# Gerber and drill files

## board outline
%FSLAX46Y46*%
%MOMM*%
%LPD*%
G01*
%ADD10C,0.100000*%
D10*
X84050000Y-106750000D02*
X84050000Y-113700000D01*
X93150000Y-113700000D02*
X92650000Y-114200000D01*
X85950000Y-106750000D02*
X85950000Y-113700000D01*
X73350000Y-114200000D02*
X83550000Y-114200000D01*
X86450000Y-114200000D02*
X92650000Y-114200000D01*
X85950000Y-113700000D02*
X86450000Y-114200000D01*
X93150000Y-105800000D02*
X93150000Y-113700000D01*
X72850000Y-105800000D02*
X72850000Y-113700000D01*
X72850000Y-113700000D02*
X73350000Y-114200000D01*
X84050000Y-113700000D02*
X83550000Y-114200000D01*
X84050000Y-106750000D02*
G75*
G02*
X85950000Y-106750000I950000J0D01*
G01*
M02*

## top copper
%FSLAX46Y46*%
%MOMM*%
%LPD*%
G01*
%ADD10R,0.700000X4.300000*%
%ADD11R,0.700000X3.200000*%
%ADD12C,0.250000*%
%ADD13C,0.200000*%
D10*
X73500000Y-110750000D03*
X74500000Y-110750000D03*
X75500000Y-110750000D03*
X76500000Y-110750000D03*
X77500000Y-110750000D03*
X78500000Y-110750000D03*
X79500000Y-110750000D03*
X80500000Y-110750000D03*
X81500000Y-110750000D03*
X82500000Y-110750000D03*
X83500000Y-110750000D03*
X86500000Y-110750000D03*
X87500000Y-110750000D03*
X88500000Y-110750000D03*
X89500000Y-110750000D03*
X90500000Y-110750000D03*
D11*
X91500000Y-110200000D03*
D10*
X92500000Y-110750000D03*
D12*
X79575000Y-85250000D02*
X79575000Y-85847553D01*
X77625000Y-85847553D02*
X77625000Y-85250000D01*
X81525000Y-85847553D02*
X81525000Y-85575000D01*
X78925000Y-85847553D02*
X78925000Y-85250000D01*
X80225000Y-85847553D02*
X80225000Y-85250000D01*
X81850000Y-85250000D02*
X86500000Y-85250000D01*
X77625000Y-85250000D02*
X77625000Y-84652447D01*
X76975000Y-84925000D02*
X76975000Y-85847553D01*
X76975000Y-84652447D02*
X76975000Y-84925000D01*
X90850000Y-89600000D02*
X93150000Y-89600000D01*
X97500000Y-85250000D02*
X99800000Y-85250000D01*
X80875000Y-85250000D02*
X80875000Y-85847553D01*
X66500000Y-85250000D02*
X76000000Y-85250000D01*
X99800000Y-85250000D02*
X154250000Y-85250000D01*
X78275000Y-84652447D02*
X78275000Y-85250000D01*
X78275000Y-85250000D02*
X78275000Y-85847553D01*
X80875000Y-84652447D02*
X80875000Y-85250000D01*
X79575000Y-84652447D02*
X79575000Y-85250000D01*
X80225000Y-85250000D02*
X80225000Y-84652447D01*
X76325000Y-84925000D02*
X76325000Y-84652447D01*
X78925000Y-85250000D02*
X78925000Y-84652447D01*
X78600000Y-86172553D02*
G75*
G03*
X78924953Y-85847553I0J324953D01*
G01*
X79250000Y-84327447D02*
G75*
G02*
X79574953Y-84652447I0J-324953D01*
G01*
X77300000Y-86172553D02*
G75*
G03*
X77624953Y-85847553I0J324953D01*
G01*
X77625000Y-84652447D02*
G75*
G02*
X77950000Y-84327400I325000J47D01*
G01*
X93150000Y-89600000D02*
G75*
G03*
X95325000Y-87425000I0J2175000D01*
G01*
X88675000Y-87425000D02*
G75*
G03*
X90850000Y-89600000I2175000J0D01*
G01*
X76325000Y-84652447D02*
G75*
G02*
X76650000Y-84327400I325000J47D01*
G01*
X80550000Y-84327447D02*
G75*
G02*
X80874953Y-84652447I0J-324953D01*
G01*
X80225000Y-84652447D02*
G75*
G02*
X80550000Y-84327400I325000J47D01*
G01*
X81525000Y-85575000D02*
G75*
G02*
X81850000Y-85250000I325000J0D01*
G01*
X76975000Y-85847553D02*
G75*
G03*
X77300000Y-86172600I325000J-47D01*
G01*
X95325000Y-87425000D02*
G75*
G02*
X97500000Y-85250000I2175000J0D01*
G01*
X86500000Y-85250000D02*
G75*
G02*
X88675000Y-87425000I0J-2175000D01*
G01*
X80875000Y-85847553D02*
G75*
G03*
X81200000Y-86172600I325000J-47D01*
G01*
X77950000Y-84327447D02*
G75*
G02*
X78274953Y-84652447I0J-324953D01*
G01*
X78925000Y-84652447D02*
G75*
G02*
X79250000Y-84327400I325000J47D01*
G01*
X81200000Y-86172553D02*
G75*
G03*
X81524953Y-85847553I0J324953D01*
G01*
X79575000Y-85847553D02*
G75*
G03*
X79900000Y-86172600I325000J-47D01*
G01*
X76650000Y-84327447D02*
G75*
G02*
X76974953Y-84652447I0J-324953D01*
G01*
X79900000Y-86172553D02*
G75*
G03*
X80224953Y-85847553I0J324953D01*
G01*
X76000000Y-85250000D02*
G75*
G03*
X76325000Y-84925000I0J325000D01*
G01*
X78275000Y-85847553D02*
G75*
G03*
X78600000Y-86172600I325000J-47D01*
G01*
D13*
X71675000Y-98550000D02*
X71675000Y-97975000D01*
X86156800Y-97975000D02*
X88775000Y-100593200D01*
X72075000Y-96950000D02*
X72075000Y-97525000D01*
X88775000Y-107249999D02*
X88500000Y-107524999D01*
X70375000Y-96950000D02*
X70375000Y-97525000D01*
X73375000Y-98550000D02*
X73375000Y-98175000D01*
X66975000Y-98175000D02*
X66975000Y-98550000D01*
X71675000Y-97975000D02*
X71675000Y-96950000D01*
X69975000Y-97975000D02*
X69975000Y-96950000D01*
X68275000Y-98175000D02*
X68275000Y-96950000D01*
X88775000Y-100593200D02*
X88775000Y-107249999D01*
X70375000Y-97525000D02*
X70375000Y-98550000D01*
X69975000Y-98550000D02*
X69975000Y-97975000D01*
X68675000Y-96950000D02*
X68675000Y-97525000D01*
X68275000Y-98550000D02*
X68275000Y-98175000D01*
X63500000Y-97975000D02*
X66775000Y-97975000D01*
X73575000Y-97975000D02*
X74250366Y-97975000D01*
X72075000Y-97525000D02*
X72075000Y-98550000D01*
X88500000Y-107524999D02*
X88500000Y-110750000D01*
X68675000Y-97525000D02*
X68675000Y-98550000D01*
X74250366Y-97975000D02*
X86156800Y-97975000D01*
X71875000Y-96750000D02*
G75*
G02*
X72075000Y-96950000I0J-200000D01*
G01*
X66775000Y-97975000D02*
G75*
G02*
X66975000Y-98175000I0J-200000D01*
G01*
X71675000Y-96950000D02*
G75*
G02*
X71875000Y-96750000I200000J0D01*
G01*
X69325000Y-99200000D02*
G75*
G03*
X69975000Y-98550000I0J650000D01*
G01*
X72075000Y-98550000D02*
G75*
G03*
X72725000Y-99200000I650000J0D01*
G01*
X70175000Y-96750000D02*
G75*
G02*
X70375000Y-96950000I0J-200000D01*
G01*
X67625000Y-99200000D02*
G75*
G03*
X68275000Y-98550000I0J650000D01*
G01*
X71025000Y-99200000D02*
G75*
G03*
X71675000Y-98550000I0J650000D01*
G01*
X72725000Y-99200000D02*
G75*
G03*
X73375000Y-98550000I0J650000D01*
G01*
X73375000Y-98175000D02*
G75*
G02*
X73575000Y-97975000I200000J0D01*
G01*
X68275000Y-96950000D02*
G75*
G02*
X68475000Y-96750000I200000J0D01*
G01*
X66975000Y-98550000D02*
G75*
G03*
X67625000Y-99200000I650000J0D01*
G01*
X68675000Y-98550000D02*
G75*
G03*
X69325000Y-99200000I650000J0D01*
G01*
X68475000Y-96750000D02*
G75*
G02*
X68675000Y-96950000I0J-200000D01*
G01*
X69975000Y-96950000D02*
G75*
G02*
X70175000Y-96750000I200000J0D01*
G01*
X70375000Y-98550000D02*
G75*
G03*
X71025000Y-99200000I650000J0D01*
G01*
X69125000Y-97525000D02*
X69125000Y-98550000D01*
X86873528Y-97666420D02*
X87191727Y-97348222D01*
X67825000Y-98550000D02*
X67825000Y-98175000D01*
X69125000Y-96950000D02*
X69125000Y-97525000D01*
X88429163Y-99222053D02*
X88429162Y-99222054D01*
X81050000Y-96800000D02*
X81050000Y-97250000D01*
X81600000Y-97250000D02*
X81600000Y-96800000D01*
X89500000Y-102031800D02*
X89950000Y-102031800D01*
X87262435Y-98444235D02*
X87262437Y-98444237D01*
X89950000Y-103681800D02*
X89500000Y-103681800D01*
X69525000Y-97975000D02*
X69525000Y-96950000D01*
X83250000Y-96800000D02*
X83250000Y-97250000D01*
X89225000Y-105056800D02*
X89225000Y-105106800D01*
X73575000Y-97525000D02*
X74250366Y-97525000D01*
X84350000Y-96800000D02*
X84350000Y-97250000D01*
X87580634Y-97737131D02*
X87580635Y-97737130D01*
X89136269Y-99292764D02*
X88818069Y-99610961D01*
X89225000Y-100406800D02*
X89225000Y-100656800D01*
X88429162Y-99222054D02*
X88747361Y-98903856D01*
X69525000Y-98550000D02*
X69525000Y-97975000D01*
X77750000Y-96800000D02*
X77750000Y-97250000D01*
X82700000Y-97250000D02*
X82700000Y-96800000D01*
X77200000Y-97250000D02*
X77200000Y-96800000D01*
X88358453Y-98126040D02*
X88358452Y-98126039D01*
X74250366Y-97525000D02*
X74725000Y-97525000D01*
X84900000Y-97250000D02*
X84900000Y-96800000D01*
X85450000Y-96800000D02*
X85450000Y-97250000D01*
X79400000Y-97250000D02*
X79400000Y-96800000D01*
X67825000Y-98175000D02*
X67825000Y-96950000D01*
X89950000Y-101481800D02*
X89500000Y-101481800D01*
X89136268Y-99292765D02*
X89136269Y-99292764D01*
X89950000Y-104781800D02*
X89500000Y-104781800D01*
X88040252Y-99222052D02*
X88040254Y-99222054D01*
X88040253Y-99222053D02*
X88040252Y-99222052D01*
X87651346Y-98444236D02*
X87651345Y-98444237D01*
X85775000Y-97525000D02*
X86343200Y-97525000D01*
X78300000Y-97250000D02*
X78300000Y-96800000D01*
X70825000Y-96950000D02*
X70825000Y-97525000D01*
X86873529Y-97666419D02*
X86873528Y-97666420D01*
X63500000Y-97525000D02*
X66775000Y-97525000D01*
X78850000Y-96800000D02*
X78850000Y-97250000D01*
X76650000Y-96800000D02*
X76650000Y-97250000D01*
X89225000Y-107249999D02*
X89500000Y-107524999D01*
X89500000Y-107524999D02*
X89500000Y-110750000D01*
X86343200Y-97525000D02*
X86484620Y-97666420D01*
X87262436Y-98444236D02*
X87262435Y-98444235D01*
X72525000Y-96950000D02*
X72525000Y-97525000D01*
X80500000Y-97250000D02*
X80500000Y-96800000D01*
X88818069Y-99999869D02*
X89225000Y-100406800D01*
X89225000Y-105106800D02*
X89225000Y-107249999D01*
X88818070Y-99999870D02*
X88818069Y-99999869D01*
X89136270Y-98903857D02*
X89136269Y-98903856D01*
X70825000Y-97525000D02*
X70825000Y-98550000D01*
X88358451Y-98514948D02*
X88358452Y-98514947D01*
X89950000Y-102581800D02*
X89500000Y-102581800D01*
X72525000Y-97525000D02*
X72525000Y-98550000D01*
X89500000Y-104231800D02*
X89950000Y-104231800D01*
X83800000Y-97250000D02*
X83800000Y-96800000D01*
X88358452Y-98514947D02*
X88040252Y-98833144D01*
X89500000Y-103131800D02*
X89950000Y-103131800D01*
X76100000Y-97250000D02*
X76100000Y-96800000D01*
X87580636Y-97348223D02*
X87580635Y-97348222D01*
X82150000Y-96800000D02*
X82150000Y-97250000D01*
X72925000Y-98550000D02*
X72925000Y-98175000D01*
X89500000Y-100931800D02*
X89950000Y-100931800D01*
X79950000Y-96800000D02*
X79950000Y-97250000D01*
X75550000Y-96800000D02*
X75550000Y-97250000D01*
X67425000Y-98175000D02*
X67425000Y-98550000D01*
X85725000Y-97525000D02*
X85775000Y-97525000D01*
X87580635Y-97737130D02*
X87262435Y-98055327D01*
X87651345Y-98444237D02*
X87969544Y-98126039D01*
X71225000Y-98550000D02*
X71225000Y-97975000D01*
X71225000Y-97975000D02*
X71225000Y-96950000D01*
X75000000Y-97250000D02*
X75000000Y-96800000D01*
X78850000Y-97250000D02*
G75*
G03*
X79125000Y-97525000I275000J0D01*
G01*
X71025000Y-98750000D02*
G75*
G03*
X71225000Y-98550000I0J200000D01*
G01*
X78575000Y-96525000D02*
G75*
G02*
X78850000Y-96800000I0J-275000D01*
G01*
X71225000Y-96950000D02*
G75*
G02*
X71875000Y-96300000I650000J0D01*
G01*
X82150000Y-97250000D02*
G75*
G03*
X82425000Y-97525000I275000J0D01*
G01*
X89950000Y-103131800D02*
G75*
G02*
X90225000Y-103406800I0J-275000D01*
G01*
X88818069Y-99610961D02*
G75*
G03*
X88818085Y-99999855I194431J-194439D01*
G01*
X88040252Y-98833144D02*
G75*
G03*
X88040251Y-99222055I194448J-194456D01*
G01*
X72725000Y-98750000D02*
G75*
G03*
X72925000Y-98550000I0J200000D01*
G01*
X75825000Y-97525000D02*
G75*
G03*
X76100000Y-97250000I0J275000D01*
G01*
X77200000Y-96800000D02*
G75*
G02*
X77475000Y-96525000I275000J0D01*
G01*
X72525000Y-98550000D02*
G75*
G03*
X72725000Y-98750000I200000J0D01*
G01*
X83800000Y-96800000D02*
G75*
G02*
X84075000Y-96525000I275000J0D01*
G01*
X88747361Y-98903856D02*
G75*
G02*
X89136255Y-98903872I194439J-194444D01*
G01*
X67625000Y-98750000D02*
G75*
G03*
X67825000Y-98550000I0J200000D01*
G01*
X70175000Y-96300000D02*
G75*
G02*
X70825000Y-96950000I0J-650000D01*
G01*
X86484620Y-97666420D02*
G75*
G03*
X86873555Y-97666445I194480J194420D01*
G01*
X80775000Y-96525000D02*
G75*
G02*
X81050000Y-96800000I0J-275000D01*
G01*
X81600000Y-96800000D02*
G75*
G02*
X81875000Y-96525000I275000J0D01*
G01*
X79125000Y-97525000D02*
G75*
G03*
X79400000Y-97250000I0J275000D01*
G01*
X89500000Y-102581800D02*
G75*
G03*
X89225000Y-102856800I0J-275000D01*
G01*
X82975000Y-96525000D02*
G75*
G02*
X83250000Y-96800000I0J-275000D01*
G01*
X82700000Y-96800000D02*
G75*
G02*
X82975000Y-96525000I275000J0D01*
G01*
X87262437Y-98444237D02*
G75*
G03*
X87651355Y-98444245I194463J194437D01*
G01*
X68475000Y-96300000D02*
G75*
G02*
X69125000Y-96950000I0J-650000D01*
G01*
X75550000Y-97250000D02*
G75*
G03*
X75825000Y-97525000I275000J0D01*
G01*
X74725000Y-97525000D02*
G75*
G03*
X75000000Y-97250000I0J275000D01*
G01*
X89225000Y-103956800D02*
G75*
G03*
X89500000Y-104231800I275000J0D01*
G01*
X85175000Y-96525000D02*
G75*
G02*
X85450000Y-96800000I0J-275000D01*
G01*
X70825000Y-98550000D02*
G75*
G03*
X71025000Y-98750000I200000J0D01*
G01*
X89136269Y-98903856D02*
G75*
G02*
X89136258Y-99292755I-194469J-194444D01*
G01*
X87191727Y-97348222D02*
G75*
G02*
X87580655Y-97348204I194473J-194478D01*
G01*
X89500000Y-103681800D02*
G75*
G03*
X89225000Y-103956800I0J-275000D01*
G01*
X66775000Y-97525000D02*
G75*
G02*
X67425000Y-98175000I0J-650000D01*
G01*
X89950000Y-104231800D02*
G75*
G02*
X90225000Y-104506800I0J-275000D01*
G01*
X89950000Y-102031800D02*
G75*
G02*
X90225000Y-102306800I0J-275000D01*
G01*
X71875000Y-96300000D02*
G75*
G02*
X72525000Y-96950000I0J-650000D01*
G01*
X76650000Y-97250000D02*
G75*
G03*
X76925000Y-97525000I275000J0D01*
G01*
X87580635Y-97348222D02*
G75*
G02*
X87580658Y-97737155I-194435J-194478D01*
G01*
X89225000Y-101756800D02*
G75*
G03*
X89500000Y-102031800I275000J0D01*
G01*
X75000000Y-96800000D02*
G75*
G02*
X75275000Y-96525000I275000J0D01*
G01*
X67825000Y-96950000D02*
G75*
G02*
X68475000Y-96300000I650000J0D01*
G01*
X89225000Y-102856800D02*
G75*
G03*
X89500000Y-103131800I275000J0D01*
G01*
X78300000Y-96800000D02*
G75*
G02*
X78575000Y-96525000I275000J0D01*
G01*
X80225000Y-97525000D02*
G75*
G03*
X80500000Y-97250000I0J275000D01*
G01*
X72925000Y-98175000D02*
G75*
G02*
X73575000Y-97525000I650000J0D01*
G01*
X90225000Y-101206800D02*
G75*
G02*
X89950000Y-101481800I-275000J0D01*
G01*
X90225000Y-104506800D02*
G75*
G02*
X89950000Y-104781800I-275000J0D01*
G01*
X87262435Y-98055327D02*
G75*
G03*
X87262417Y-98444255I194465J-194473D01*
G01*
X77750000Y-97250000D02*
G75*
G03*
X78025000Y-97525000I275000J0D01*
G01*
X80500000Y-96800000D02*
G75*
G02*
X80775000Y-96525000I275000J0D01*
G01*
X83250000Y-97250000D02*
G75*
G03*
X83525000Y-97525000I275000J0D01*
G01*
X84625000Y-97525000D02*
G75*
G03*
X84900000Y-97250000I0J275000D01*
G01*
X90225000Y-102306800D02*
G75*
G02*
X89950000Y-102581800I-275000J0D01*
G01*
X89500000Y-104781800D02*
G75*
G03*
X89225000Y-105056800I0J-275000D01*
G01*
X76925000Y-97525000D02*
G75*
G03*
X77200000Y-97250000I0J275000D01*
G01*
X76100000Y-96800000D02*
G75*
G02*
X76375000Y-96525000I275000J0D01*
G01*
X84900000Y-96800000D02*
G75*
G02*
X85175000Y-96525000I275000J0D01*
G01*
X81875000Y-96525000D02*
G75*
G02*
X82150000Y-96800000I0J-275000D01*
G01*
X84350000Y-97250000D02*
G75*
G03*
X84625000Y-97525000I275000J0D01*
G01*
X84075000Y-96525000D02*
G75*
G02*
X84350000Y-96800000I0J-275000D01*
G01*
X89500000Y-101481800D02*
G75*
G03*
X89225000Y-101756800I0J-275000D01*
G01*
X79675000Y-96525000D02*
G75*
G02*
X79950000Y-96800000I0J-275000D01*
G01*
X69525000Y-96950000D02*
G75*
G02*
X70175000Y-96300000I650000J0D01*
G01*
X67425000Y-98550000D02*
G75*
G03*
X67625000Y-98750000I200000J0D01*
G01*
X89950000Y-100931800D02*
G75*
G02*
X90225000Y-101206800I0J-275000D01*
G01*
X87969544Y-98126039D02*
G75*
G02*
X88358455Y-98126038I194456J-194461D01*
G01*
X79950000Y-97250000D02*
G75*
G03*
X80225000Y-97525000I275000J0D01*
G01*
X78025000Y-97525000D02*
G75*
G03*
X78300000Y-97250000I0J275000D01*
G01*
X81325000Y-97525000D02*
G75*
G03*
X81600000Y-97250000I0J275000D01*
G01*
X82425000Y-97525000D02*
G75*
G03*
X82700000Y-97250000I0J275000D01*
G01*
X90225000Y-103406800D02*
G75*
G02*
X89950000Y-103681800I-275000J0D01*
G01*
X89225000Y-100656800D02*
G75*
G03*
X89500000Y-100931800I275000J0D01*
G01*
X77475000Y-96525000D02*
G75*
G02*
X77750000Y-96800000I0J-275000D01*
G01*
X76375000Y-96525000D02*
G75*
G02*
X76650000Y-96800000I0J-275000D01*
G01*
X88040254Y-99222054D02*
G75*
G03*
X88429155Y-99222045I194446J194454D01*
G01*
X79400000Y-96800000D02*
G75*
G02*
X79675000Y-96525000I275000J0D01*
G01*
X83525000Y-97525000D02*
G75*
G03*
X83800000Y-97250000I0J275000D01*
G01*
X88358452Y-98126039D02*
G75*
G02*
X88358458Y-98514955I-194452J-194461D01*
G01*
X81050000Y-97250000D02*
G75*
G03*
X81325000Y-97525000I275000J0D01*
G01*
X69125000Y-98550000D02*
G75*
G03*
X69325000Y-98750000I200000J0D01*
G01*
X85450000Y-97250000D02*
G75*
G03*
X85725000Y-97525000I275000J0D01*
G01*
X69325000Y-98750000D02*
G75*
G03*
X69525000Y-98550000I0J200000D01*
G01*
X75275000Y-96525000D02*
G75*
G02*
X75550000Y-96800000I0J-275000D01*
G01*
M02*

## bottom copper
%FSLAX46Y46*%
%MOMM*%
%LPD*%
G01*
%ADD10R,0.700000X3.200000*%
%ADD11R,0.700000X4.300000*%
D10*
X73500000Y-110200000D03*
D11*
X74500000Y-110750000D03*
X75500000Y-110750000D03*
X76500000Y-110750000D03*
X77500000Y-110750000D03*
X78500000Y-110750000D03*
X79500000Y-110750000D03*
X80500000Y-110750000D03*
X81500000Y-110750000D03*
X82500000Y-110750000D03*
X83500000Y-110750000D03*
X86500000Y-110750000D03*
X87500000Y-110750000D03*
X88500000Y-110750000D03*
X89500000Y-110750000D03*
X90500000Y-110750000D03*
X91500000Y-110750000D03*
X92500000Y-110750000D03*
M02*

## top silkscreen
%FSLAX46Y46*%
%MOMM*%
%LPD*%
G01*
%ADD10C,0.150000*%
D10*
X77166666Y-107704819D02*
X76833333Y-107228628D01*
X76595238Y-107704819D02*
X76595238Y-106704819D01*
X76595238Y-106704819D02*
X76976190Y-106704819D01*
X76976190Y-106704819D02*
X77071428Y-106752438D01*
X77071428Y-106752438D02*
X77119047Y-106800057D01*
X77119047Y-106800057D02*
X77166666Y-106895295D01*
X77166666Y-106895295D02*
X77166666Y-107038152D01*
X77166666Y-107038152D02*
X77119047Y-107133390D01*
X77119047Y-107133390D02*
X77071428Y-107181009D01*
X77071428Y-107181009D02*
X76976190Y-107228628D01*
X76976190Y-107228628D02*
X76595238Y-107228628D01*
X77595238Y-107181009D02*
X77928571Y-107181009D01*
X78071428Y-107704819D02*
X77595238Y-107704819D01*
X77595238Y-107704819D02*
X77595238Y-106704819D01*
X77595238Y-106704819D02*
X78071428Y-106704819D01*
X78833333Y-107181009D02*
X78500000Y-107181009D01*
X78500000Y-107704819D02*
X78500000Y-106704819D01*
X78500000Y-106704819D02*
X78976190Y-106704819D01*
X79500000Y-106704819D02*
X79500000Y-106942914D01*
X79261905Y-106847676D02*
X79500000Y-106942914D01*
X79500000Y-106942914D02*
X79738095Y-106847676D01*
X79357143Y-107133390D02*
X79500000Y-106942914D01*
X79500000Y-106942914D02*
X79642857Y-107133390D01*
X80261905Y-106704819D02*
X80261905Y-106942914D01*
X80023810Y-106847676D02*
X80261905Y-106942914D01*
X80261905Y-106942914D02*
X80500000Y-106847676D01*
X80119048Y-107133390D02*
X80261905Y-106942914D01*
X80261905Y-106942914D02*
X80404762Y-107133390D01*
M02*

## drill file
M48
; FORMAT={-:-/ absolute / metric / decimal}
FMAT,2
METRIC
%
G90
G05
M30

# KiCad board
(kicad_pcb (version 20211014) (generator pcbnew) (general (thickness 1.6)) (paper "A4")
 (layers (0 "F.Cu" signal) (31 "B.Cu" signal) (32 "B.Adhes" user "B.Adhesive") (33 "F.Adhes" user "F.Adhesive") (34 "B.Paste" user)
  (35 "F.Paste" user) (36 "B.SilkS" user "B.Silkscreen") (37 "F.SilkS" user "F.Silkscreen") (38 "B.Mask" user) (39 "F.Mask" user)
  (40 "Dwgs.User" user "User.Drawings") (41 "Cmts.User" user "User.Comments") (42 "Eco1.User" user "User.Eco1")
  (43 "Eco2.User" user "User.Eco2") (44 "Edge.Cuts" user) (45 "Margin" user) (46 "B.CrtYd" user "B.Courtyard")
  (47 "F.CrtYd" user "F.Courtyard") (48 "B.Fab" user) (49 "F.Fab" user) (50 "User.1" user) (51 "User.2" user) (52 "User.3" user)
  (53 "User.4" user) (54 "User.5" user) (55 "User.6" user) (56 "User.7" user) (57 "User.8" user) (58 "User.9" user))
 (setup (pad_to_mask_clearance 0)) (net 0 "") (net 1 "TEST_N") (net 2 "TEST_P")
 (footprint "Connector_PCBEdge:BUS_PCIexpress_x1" (layer "F.Cu") (at 73.5 110.75)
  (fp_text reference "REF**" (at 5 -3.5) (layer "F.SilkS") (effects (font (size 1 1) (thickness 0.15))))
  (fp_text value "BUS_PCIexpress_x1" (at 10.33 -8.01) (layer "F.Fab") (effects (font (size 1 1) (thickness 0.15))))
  (fp_line (start 10.55 -4) (end 10.55 2.95) (layer "Edge.Cuts") (width 0.1))
  (fp_line (start 19.65 2.95) (end 19.15 3.45) (layer "Edge.Cuts") (width 0.1))
  (fp_line (start 12.45 -4) (end 12.45 2.95) (layer "Edge.Cuts") (width 0.1))
  (fp_line (start -0.15 3.45) (end 10.05 3.45) (layer "Edge.Cuts") (width 0.1))
  (fp_line (start 12.95 3.45) (end 19.15 3.45) (layer "Edge.Cuts") (width 0.1))
  (fp_line (start 12.45 2.95) (end 12.95 3.45) (layer "Edge.Cuts") (width 0.1))
  (fp_line (start 19.65 -4.95) (end 19.65 2.95) (layer "Edge.Cuts") (width 0.1))
  (fp_line (start -0.65 -4.95) (end -0.65 2.95) (layer "Edge.Cuts") (width 0.1))
  (fp_line (start -0.65 2.95) (end -0.15 3.45) (layer "Edge.Cuts") (width 0.1))
  (fp_line (start 10.55 2.95) (end 10.05 3.45) (layer "Edge.Cuts") (width 0.1))
  (fp_arc (start 10.55 -4) (mid 11.5 -4.95) (end 12.45 -4) (layer "Edge.Cuts") (width 0.1))
  (pad "A1" connect rect locked (at 0 -0.55) (size 0.7 3.2) (layers "B.Cu" "B.Mask"))
  (pad "A2" connect rect locked (at 1 0) (size 0.7 4.3) (layers "B.Cu" "B.Mask"))
  (pad "A3" connect rect locked (at 2 0) (size 0.7 4.3) (layers "B.Cu" "B.Mask"))
  (pad "A4" connect rect locked (at 3 0) (size 0.7 4.3) (layers "B.Cu" "B.Mask"))
  (pad "A5" connect rect locked (at 4 0) (size 0.7 4.3) (layers "B.Cu" "B.Mask"))
  (pad "A6" connect rect locked (at 5 0) (size 0.7 4.3) (layers "B.Cu" "B.Mask"))
  (pad "A7" connect rect locked (at 6 0) (size 0.7 4.3) (layers "B.Cu" "B.Mask"))
  (pad "A8" connect rect locked (at 7 0) (size 0.7 4.3) (layers "B.Cu" "B.Mask"))
  (pad "A9" connect rect locked (at 8 0) (size 0.7 4.3) (layers "B.Cu" "B.Mask"))
  (pad "A10" connect rect locked (at 9 0) (size 0.7 4.3) (layers "B.Cu" "B.Mask"))
  (pad "A11" connect rect locked (at 10 0) (size 0.7 4.3) (layers "B.Cu" "B.Mask"))
  (pad "A12" connect rect locked (at 13 0) (size 0.7 4.3) (layers "B.Cu" "B.Mask"))
  (pad "A13" connect rect locked (at 14 0) (size 0.7 4.3) (layers "B.Cu" "B.Mask"))
  (pad "A14" connect rect locked (at 15 0) (size 0.7 4.3) (layers "B.Cu" "B.Mask"))
  (pad "A15" connect rect locked (at 16 0) (size 0.7 4.3) (layers "B.Cu" "B.Mask"))
  (pad "A16" connect rect locked (at 17 0) (size 0.7 4.3) (layers "B.Cu" "B.Mask"))
  (pad "A17" connect rect locked (at 18 0) (size 0.7 4.3) (layers "B.Cu" "B.Mask"))
  (pad "A18" connect rect locked (at 19 0) (size 0.7 4.3) (layers "B.Cu" "B.Mask"))
  (pad "B1" connect rect locked (at 0 0) (size 0.7 4.3) (layers "F.Cu" "F.Mask"))
  (pad "B2" connect rect locked (at 1 0) (size 0.7 4.3) (layers "F.Cu" "F.Mask"))
  (pad "B3" connect rect locked (at 2 0) (size 0.7 4.3) (layers "F.Cu" "F.Mask"))
  (pad "B4" connect rect locked (at 3 0) (size 0.7 4.3) (layers "F.Cu" "F.Mask"))
  (pad "B5" connect rect locked (at 4 0) (size 0.7 4.3) (layers "F.Cu" "F.Mask"))
  (pad "B6" connect rect locked (at 5 0) (size 0.7 4.3) (layers "F.Cu" "F.Mask"))
  (pad "B7" connect rect locked (at 6 0) (size 0.7 4.3) (layers "F.Cu" "F.Mask"))
  (pad "B8" connect rect locked (at 7 0) (size 0.7 4.3) (layers "F.Cu" "F.Mask"))
  (pad "B9" connect rect locked (at 8 0) (size 0.7 4.3) (layers "F.Cu" "F.Mask"))
  (pad "B10" connect rect locked (at 9 0) (size 0.7 4.3) (layers "F.Cu" "F.Mask"))
  (pad "B11" connect rect locked (at 10 0) (size 0.7 4.3) (layers "F.Cu" "F.Mask"))
  (pad "B12" connect rect locked (at 13 0) (size 0.7 4.3) (layers "F.Cu" "F.Mask"))
  (pad "B13" connect rect locked (at 14 0) (size 0.7 4.3) (layers "F.Cu" "F.Mask"))
  (pad "B14" connect rect locked (at 15 0) (size 0.7 4.3) (layers "F.Cu" "F.Mask") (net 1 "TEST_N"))
  (pad "B15" connect rect locked (at 16 0) (size 0.7 4.3) (layers "F.Cu" "F.Mask") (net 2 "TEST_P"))
  (pad "B16" connect rect locked (at 17 0) (size 0.7 4.3) (layers "F.Cu" "F.Mask"))
  (pad "B17" connect rect locked (at 18 -0.55) (size 0.7 3.2) (layers "F.Cu" "F.Mask"))
  (pad "B18" connect rect locked (at 19 0) (size 0.7 4.3) (layers "F.Cu" "F.Mask")))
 (segment (start 79.575 85.25) (end 79.575 85.847553) (width 0.25) (layer "F.Cu") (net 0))
 (segment (start 77.625 85.847553) (end 77.625 85.25) (width 0.25) (layer "F.Cu") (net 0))
 (segment (start 81.525 85.847553) (end 81.525 85.575) (width 0.25) (layer "F.Cu") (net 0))
 (segment (start 78.925 85.847553) (end 78.925 85.25) (width 0.25) (layer "F.Cu") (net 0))
 (segment (start 80.225 85.847553) (end 80.225 85.25) (width 0.25) (layer "F.Cu") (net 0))
 (segment (start 81.85 85.25) (end 86.5 85.25) (width 0.25) (layer "F.Cu") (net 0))
 (segment (start 77.625 85.25) (end 77.625 84.652447) (width 0.25) (layer "F.Cu") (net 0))
 (segment (start 76.975 84.925) (end 76.975 85.847553) (width 0.25) (layer "F.Cu") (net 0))
 (segment (start 76.975 84.652447) (end 76.975 84.925) (width 0.25) (layer "F.Cu") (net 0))
 (segment (start 90.85 89.6) (end 93.15 89.6) (width 0.25) (layer "F.Cu") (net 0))
 (segment (start 97.5 85.25) (end 99.8 85.25) (width 0.25) (layer "F.Cu") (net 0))
 (segment (start 80.875 85.25) (end 80.875 85.847553) (width 0.25) (layer "F.Cu") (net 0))
 (segment (start 66.5 85.25) (end 76 85.25) (width 0.25) (layer "F.Cu") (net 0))
 (segment (start 99.8 85.25) (end 154.25 85.25) (width 0.25) (layer "F.Cu") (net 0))
 (segment (start 78.275 84.652447) (end 78.275 85.25) (width 0.25) (layer "F.Cu") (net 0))
 (segment (start 78.275 85.25) (end 78.275 85.847553) (width 0.25) (layer "F.Cu") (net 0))
 (segment (start 80.875 84.652447) (end 80.875 85.25) (width 0.25) (layer "F.Cu") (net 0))
 (segment (start 79.575 84.652447) (end 79.575 85.25) (width 0.25) (layer "F.Cu") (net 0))
 (segment (start 80.225 85.25) (end 80.225 84.652447) (width 0.25) (layer "F.Cu") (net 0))
 (segment (start 76.325 84.925) (end 76.325 84.652447) (width 0.25) (layer "F.Cu") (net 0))
 (segment (start 78.925 85.25) (end 78.925 84.652447) (width 0.25) (layer "F.Cu") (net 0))
 (arc (start 78.6 86.172553) (mid 78.82981 86.077363) (end 78.925 85.847553) (width 0.25) (layer "F.Cu") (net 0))
 (arc (start 79.25 84.327447) (mid 79.47981 84.422637) (end 79.575 84.652447) (width 0.25) (layer "F.Cu") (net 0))
 (arc (start 77.3 86.172553) (mid 77.52981 86.077363) (end 77.625 85.847553) (width 0.25) (layer "F.Cu") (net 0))
 (arc (start 77.625 84.652447) (mid 77.72019 84.422637) (end 77.95 84.327447) (width 0.25) (layer "F.Cu") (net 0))
 (arc (start 93.15 89.6) (mid 94.687957 88.962957) (end 95.325 87.425) (width 0.25) (layer "F.Cu") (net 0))
 (arc (start 88.675 87.425) (mid 89.312043 88.962957) (end 90.85 89.6) (width 0.25) (layer "F.Cu") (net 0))
 (arc (start 76.325 84.652447) (mid 76.42019 84.422637) (end 76.65 84.327447) (width 0.25) (layer "F.Cu") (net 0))
 (arc (start 80.55 84.327447) (mid 80.77981 84.422637) (end 80.875 84.652447) (width 0.25) (layer "F.Cu") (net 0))
 (arc (start 80.225 84.652447) (mid 80.32019 84.422637) (end 80.55 84.327447) (width 0.25) (layer "F.Cu") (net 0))
 (arc (start 81.525 85.575) (mid 81.62019 85.34519) (end 81.85 85.25) (width 0.25) (layer "F.Cu") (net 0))
 (arc (start 76.975 85.847553) (mid 77.07019 86.077363) (end 77.3 86.172553) (width 0.25) (layer "F.Cu") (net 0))
 (arc (start 95.325 87.425) (mid 95.962043 85.887043) (end 97.5 85.25) (width 0.25) (layer "F.Cu") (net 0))
 (arc (start 86.5 85.25) (mid 88.037957 85.887043) (end 88.675 87.425) (width 0.25) (layer "F.Cu") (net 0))
 (arc (start 80.875 85.847553) (mid 80.97019 86.077363) (end 81.2 86.172553) (width 0.25) (layer "F.Cu") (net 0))
 (arc (start 77.95 84.327447) (mid 78.17981 84.422637) (end 78.275 84.652447) (width 0.25) (layer "F.Cu") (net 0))
 (arc (start 78.925 84.652447) (mid 79.02019 84.422637) (end 79.25 84.327447) (width 0.25) (layer "F.Cu") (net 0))
 (arc (start 81.2 86.172553) (mid 81.42981 86.077363) (end 81.525 85.847553) (width 0.25) (layer "F.Cu") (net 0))
 (arc (start 79.575 85.847553) (mid 79.67019 86.077363) (end 79.9 86.172553) (width 0.25) (layer "F.Cu") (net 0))
 (arc (start 76.65 84.327447) (mid 76.87981 84.422637) (end 76.975 84.652447) (width 0.25) (layer "F.Cu") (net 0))
 (arc (start 79.9 86.172553) (mid 80.12981 86.077363) (end 80.225 85.847553) (width 0.25) (layer "F.Cu") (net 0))
 (arc (start 76 85.25) (mid 76.22981 85.15481) (end 76.325 84.925) (width 0.25) (layer "F.Cu") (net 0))
 (arc (start 78.275 85.847553) (mid 78.37019 86.077363) (end 78.6 86.172553) (width 0.25) (layer "F.Cu") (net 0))
 (segment (start 71.675 98.55) (end 71.675 97.975) (width 0.2) (layer "F.Cu") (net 1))
 (segment (start 86.1568 97.975) (end 88.775 100.5932) (width 0.2) (layer "F.Cu") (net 1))
 (segment (start 72.075 96.95) (end 72.075 97.525) (width 0.2) (layer "F.Cu") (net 1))
 (segment (start 88.775 107.249999) (end 88.5 107.524999) (width 0.2) (layer "F.Cu") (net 1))
 (segment (start 70.375 96.95) (end 70.375 97.525) (width 0.2) (layer "F.Cu") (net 1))
 (segment (start 73.375 98.55) (end 73.375 98.175) (width 0.2) (layer "F.Cu") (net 1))
 (segment (start 66.975 98.175) (end 66.975 98.55) (width 0.2) (layer "F.Cu") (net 1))
 (segment (start 71.675 97.975) (end 71.675 96.95) (width 0.2) (layer "F.Cu") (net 1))
 (segment (start 69.975 97.975) (end 69.975 96.95) (width 0.2) (layer "F.Cu") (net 1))
 (segment (start 68.275 98.175) (end 68.275 96.95) (width 0.2) (layer "F.Cu") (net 1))
 (segment (start 88.775 100.5932) (end 88.775 107.249999) (width 0.2) (layer "F.Cu") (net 1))
 (segment (start 70.375 97.525) (end 70.375 98.55) (width 0.2) (layer "F.Cu") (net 1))
 (segment (start 69.975 98.55) (end 69.975 97.975) (width 0.2) (layer "F.Cu") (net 1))
 (segment (start 68.675 96.95) (end 68.675 97.525) (width 0.2) (layer "F.Cu") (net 1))
 (segment (start 68.275 98.55) (end 68.275 98.175) (width 0.2) (layer "F.Cu") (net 1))
 (segment (start 63.5 97.975) (end 66.775 97.975) (width 0.2) (layer "F.Cu") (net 1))
 (segment (start 73.575 97.975) (end 74.250366 97.975) (width 0.2) (layer "F.Cu") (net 1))
 (segment (start 72.075 97.525) (end 72.075 98.55) (width 0.2) (layer "F.Cu") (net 1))
 (segment (start 88.5 107.524999) (end 88.5 110.75) (width 0.2) (layer "F.Cu") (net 1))
 (segment (start 68.675 97.525) (end 68.675 98.55) (width 0.2) (layer "F.Cu") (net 1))
 (segment (start 74.250366 97.975) (end 86.1568 97.975) (width 0.2) (layer "F.Cu") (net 1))
 (arc (start 71.875 96.75) (mid 72.016421 96.808579) (end 72.075 96.95) (width 0.2) (layer "F.Cu") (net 1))
 (arc (start 66.775 97.975) (mid 66.916421 98.033579) (end 66.975 98.175) (width 0.2) (layer "F.Cu") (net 1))
 (arc (start 71.675 96.95) (mid 71.733579 96.808579) (end 71.875 96.75) (width 0.2) (layer "F.Cu") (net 1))
 (arc (start 69.325 99.2) (mid 69.784619 99.009619) (end 69.975 98.55) (width 0.2) (layer "F.Cu") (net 1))
 (arc (start 72.075 98.55) (mid 72.265381 99.009619) (end 72.725 99.2) (width 0.2) (layer "F.Cu") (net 1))
 (arc (start 70.175 96.75) (mid 70.316421 96.808579) (end 70.375 96.95) (width 0.2) (layer "F.Cu") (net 1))
 (arc (start 67.625 99.2) (mid 68.084619 99.009619) (end 68.275 98.55) (width 0.2) (layer "F.Cu") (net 1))
 (arc (start 71.025 99.2) (mid 71.484619 99.009619) (end 71.675 98.55) (width 0.2) (layer "F.Cu") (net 1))
 (arc (start 72.725 99.2) (mid 73.184619 99.009619) (end 73.375 98.55) (width 0.2) (layer "F.Cu") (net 1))
 (arc (start 73.375 98.175) (mid 73.433579 98.033579) (end 73.575 97.975) (width 0.2) (layer "F.Cu") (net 1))
 (arc (start 68.275 96.95) (mid 68.333579 96.808579) (end 68.475 96.75) (width 0.2) (layer "F.Cu") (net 1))
 (arc (start 66.975 98.55) (mid 67.165381 99.009619) (end 67.625 99.2) (width 0.2) (layer "F.Cu") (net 1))
 (arc (start 68.675 98.55) (mid 68.865381 99.009619) (end 69.325 99.2) (width 0.2) (layer "F.Cu") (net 1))
 (arc (start 68.475 96.75) (mid 68.616421 96.808579) (end 68.675 96.95) (width 0.2) (layer "F.Cu") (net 1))
 (arc (start 69.975 96.95) (mid 70.033579 96.808579) (end 70.175 96.75) (width 0.2) (layer "F.Cu") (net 1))
 (arc (start 70.375 98.55) (mid 70.565381 99.009619) (end 71.025 99.2) (width 0.2) (layer "F.Cu") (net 1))
 (segment (start 69.125 97.525) (end 69.125 98.55) (width 0.2) (layer "F.Cu") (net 2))
 (segment (start 86.873528 97.66642) (end 87.191727 97.348222) (width 0.2) (layer "F.Cu") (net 2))
 (segment (start 67.825 98.55) (end 67.825 98.175) (width 0.2) (layer "F.Cu") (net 2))
 (segment (start 69.125 96.95) (end 69.125 97.525) (width 0.2) (layer "F.Cu") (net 2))
 (segment (start 88.429163 99.222053) (end 88.429162 99.222054) (width 0.2) (layer "F.Cu") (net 2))
 (segment locked (start 81.05 96.8) (end 81.05 97.25) (width 0.2) (layer "F.Cu") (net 2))
 (segment locked (start 81.6 97.25) (end 81.6 96.8) (width 0.2) (layer "F.Cu") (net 2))
 (segment (start 89.5 102.0318) (end 89.95 102.0318) (width 0.2) (layer "F.Cu") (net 2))
 (segment (start 87.262435 98.444235) (end 87.262437 98.444237) (width 0.2) (layer "F.Cu") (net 2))
 (segment (start 89.95 103.6818) (end 89.5 103.6818) (width 0.2) (layer "F.Cu") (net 2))
 (segment (start 69.525 97.975) (end 69.525 96.95) (width 0.2) (layer "F.Cu") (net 2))
 (segment locked (start 83.25 96.8) (end 83.25 97.25) (width 0.2) (layer "F.Cu") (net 2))
 (segment (start 89.225 105.0568) (end 89.225 105.1068) (width 0.2) (layer "F.Cu") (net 2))
 (segment (start 73.575 97.525) (end 74.250366 97.525) (width 0.2) (layer "F.Cu") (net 2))
 (segment locked (start 84.35 96.8) (end 84.35 97.25) (width 0.2) (layer "F.Cu") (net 2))
 (segment (start 87.580634 97.737131) (end 87.580635 97.73713) (width 0.2) (layer "F.Cu") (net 2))
 (segment (start 89.136269 99.292764) (end 88.818069 99.610961) (width 0.2) (layer "F.Cu") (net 2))
 (segment (start 89.225 100.4068) (end 89.225 100.6568) (width 0.2) (layer "F.Cu") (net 2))
 (segment (start 88.429162 99.222054) (end 88.747361 98.903856) (width 0.2) (layer "F.Cu") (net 2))
 (segment (start 69.525 98.55) (end 69.525 97.975) (width 0.2) (layer "F.Cu") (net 2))
 (segment locked (start 77.75 96.8) (end 77.75 97.25) (width 0.2) (layer "F.Cu") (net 2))
 (segment locked (start 82.7 97.25) (end 82.7 96.8) (width 0.2) (layer "F.Cu") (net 2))
 (segment locked (start 77.2 97.25) (end 77.2 96.8) (width 0.2) (layer "F.Cu") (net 2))
 (segment (start 88.358453 98.12604) (end 88.358452 98.126039) (width 0.2) (layer "F.Cu") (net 2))
 (segment locked (start 74.250366 97.525) (end 74.725 97.525) (width 0.2) (layer "F.Cu") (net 2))
 (segment locked (start 84.9 97.25) (end 84.9 96.8) (width 0.2) (layer "F.Cu") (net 2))
 (segment locked (start 85.45 96.8) (end 85.45 97.25) (width 0.2) (layer "F.Cu") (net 2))
 (segment locked (start 79.4 97.25) (end 79.4 96.8) (width 0.2) (layer "F.Cu") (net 2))
 (segment (start 67.825 98.175) (end 67.825 96.95) (width 0.2) (layer "F.Cu") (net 2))
 (segment (start 89.95 101.4818) (end 89.5 101.4818) (width 0.2) (layer "F.Cu") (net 2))
 (segment (start 89.136268 99.292765) (end 89.136269 99.292764) (width 0.2) (layer "F.Cu") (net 2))
 (segment (start 89.95 104.7818) (end 89.5 104.7818) (width 0.2) (layer "F.Cu") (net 2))
 (segment (start 88.040252 99.222052) (end 88.040254 99.222054) (width 0.2) (layer "F.Cu") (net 2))
 (segment (start 88.040253 99.222053) (end 88.040252 99.222052) (width 0.2) (layer "F.Cu") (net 2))
 (segment (start 87.651346 98.444236) (end 87.651345 98.444237) (width 0.2) (layer "F.Cu") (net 2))
 (segment (start 85.775 97.525) (end 86.3432 97.525) (width 0.2) (layer "F.Cu") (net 2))
 (segment locked (start 78.3 97.25) (end 78.3 96.8) (width 0.2) (layer "F.Cu") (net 2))
 (segment (start 70.825 96.95) (end 70.825 97.525) (width 0.2) (layer "F.Cu") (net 2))
 (segment (start 86.873529 97.666419) (end 86.873528 97.66642) (width 0.2) (layer "F.Cu") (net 2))
 (segment (start 63.5 97.525) (end 66.775 97.525) (width 0.2) (layer "F.Cu") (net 2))
 (segment locked (start 78.85 96.8) (end 78.85 97.25) (width 0.2) (layer "F.Cu") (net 2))
 (segment locked (start 76.65 96.8) (end 76.65 97.25) (width 0.2) (layer "F.Cu") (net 2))
 (segment (start 89.225 107.249999) (end 89.5 107.524999) (width 0.2) (layer "F.Cu") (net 2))
 (segment (start 89.5 107.524999) (end 89.5 110.75) (width 0.2) (layer "F.Cu") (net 2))
 (segment (start 86.3432 97.525) (end 86.48462 97.66642) (width 0.2) (layer "F.Cu") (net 2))
 (segment (start 87.262436 98.444236) (end 87.262435 98.444235) (width 0.2) (layer "F.Cu") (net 2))
 (segment (start 72.525 96.95) (end 72.525 97.525) (width 0.2) (layer "F.Cu") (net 2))
 (segment locked (start 80.5 97.25) (end 80.5 96.8) (width 0.2) (layer "F.Cu") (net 2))
 (segment (start 88.818069 99.999869) (end 89.225 100.4068) (width 0.2) (layer "F.Cu") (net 2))
 (segment (start 89.225 105.1068) (end 89.225 107.249999) (width 0.2) (layer "F.Cu") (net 2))
 (segment (start 88.81807 99.99987) (end 88.818069 99.999869) (width 0.2) (layer "F.Cu") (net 2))
 (segment (start 89.13627 98.903857) (end 89.136269 98.903856) (width 0.2) (layer "F.Cu") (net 2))
 (segment (start 70.825 97.525) (end 70.825 98.55) (width 0.2) (layer "F.Cu") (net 2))
 (segment (start 88.358451 98.514948) (end 88.358452 98.514947) (width 0.2) (layer "F.Cu") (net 2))
 (segment (start 89.95 102.5818) (end 89.5 102.5818) (width 0.2) (layer "F.Cu") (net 2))
 (segment (start 72.525 97.525) (end 72.525 98.55) (width 0.2) (layer "F.Cu") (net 2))
 (segment (start 89.5 104.2318) (end 89.95 104.2318) (width 0.2) (layer "F.Cu") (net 2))
 (segment locked (start 83.8 97.25) (end 83.8 96.8) (width 0.2) (layer "F.Cu") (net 2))
 (segment (start 88.358452 98.514947) (end 88.040252 98.833144) (width 0.2) (layer "F.Cu") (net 2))
 (segment (start 89.5 103.1318) (end 89.95 103.1318) (width 0.2) (layer "F.Cu") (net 2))
 (segment locked (start 76.1 97.25) (end 76.1 96.8) (width 0.2) (layer "F.Cu") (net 2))
 (segment (start 87.580636 97.348223) (end 87.580635 97.348222) (width 0.2) (layer "F.Cu") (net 2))
 (segment locked (start 82.15 96.8) (end 82.15 97.25) (width 0.2) (layer "F.Cu") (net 2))
 (segment (start 72.925 98.55) (end 72.925 98.175) (width 0.2) (layer "F.Cu") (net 2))
 (segment (start 89.5 100.9318) (end 89.95 100.9318) (width 0.2) (layer "F.Cu") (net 2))
 (segment locked (start 79.95 96.8) (end 79.95 97.25) (width 0.2) (layer "F.Cu") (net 2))
 (segment locked (start 75.55 96.8) (end 75.55 97.25) (width 0.2) (layer "F.Cu") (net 2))
 (segment (start 67.425 98.175) (end 67.425 98.55) (width 0.2) (layer "F.Cu") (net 2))
 (segment locked (start 85.725 97.525) (end 85.775 97.525) (width 0.2) (layer "F.Cu") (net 2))
 (segment (start 87.580635 97.73713) (end 87.262435 98.055327) (width 0.2) (layer "F.Cu") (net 2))
 (segment (start 87.651345 98.444237) (end 87.969544 98.126039) (width 0.2) (layer "F.Cu") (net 2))
 (segment (start 71.225 98.55) (end 71.225 97.975) (width 0.2) (layer "F.Cu") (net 2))
 (segment (start 71.225 97.975) (end 71.225 96.95) (width 0.2) (layer "F.Cu") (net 2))
 (segment locked (start 75 97.25) (end 75 96.8) (width 0.2) (layer "F.Cu") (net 2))
 (arc locked (start 78.85 97.25) (mid 78.930546 97.444454) (end 79.125 97.525) (width 0.2) (layer "F.Cu") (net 2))
 (arc (start 71.025 98.75) (mid 71.166421 98.691421) (end 71.225 98.55) (width 0.2) (layer "F.Cu") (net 2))
 (arc locked (start 78.575 96.525) (mid 78.769454 96.605546) (end 78.85 96.8) (width 0.2) (layer "F.Cu") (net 2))
 (arc (start 71.225 96.95) (mid 71.415381 96.490381) (end 71.875 96.3) (width 0.2) (layer "F.Cu") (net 2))
 (arc locked (start 82.15 97.25) (mid 82.230546 97.444454) (end 82.425 97.525) (width 0.2) (layer "F.Cu") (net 2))
 (arc (start 89.95 103.1318) (mid 90.144454 103.212346) (end 90.225 103.4068) (width 0.2) (layer "F.Cu") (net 2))
 (arc (start 88.818069 99.610961) (mid 88.737524 99.805416) (end 88.81807 99.99987) (width 0.2) (layer "F.Cu") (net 2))
 (arc (start 88.040252 98.833144) (mid 87.959707 99.027599) (end 88.040253 99.222053) (width 0.2) (layer "F.Cu") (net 2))
 (arc (start 72.725 98.75) (mid 72.866421 98.691421) (end 72.925 98.55) (width 0.2) (layer "F.Cu") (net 2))
 (arc locked (start 75.825 97.525) (mid 76.019454 97.444454) (end 76.1 97.25) (width 0.2) (layer "F.Cu") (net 2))
 (arc locked (start 77.2 96.8) (mid 77.280546 96.605546) (end 77.475 96.525) (width 0.2) (layer "F.Cu") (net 2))
 (arc (start 72.525 98.55) (mid 72.583579 98.691421) (end 72.725 98.75) (width 0.2) (layer "F.Cu") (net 2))
 (arc locked (start 83.8 96.8) (mid 83.880546 96.605546) (end 84.075 96.525) (width 0.2) (layer "F.Cu") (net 2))
 (arc (start 88.747361 98.903856) (mid 88.941816 98.823311) (end 89.13627 98.903857) (width 0.2) (layer "F.Cu") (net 2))
 (arc (start 67.625 98.75) (mid 67.766421 98.691421) (end 67.825 98.55) (width 0.2) (layer "F.Cu") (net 2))
 (arc (start 70.175 96.3) (mid 70.634619 96.490381) (end 70.825 96.95) (width 0.2) (layer "F.Cu") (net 2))
 (arc (start 86.48462 97.66642) (mid 86.679075 97.746965) (end 86.873529 97.666419) (width 0.2) (layer "F.Cu") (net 2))
 (arc locked (start 80.775 96.525) (mid 80.969454 96.605546) (end 81.05 96.8) (width 0.2) (layer "F.Cu") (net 2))
 (arc locked (start 81.6 96.8) (mid 81.680546 96.605546) (end 81.875 96.525) (width 0.2) (layer "F.Cu") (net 2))
 (arc locked (start 79.125 97.525) (mid 79.319454 97.444454) (end 79.4 97.25) (width 0.2) (layer "F.Cu") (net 2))
 (arc (start 89.5 102.5818) (mid 89.305546 102.662346) (end 89.225 102.8568) (width 0.2) (layer "F.Cu") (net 2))
 (arc locked (start 82.975 96.525) (mid 83.169454 96.605546) (end 83.25 96.8) (width 0.2) (layer "F.Cu") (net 2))
 (arc locked (start 82.7 96.8) (mid 82.780546 96.605546) (end 82.975 96.525) (width 0.2) (layer "F.Cu") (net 2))
 (arc (start 87.262437 98.444237) (mid 87.456892 98.524782) (end 87.651346 98.444236) (width 0.2) (layer "F.Cu") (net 2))
 (arc (start 68.475 96.3) (mid 68.934619 96.490381) (end 69.125 96.95) (width 0.2) (layer "F.Cu") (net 2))
 (arc locked (start 75.55 97.25) (mid 75.630546 97.444454) (end 75.825 97.525) (width 0.2) (layer "F.Cu") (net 2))
 (arc locked (start 74.725 97.525) (mid 74.919454 97.444454) (end 75 97.25) (width 0.2) (layer "F.Cu") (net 2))
 (arc (start 89.225 103.9568) (mid 89.305546 104.151254) (end 89.5 104.2318) (width 0.2) (layer "F.Cu") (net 2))
 (arc locked (start 85.175 96.525) (mid 85.369454 96.605546) (end 85.45 96.8) (width 0.2) (layer "F.Cu") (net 2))
 (arc (start 70.825 98.55) (mid 70.883579 98.691421) (end 71.025 98.75) (width 0.2) (layer "F.Cu") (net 2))
 (arc (start 89.136269 98.903856) (mid 89.216814 99.098311) (end 89.136268 99.292765) (width 0.2) (layer "F.Cu") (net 2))
 (arc (start 87.191727 97.348222) (mid 87.386182 97.267677) (end 87.580636 97.348223) (width 0.2) (layer "F.Cu") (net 2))
 (arc (start 89.5 103.6818) (mid 89.305546 103.762346) (end 89.225 103.9568) (width 0.2) (layer "F.Cu") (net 2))
 (arc (start 66.775 97.525) (mid 67.234619 97.715381) (end 67.425 98.175) (width 0.2) (layer "F.Cu") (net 2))
 (arc (start 89.95 104.2318) (mid 90.144454 104.312346) (end 90.225 104.5068) (width 0.2) (layer "F.Cu") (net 2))
 (arc (start 89.95 102.0318) (mid 90.144454 102.112346) (end 90.225 102.3068) (width 0.2) (layer "F.Cu") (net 2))
 (arc (start 71.875 96.3) (mid 72.334619 96.490381) (end 72.525 96.95) (width 0.2) (layer "F.Cu") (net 2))
 (arc locked (start 76.65 97.25) (mid 76.730546 97.444454) (end 76.925 97.525) (width 0.2) (layer "F.Cu") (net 2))
 (arc (start 87.580635 97.348222) (mid 87.66118 97.542677) (end 87.580634 97.737131) (width 0.2) (layer "F.Cu") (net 2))
 (arc (start 89.225 101.7568) (mid 89.305546 101.951254) (end 89.5 102.0318) (width 0.2) (layer "F.Cu") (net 2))
 (arc locked (start 75 96.8) (mid 75.080546 96.605546) (end 75.275 96.525) (width 0.2) (layer "F.Cu") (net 2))
 (arc (start 67.825 96.95) (mid 68.015381 96.490381) (end 68.475 96.3) (width 0.2) (layer "F.Cu") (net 2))
 (arc (start 89.225 102.8568) (mid 89.305546 103.051254) (end 89.5 103.1318) (width 0.2) (layer "F.Cu") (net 2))
 (arc locked (start 78.3 96.8) (mid 78.380546 96.605546) (end 78.575 96.525) (width 0.2) (layer "F.Cu") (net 2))
 (arc locked (start 80.225 97.525) (mid 80.419454 97.444454) (end 80.5 97.25) (width 0.2) (layer "F.Cu") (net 2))
 (arc (start 72.925 98.175) (mid 73.115381 97.715381) (end 73.575 97.525) (width 0.2) (layer "F.Cu") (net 2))
 (arc (start 90.225 101.2068) (mid 90.144454 101.401254) (end 89.95 101.4818) (width 0.2) (layer "F.Cu") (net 2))
 (arc (start 90.225 104.5068) (mid 90.144454 104.701254) (end 89.95 104.7818) (width 0.2) (layer "F.Cu") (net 2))
 (arc (start 87.262435 98.055327) (mid 87.18189 98.249782) (end 87.262436 98.444236) (width 0.2) (layer "F.Cu") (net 2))
 (arc locked (start 77.75 97.25) (mid 77.830546 97.444454) (end 78.025 97.525) (width 0.2) (layer "F.Cu") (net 2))
 (arc locked (start 80.5 96.8) (mid 80.580546 96.605546) (end 80.775 96.525) (width 0.2) (layer "F.Cu") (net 2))
 (arc locked (start 83.25 97.25) (mid 83.330546 97.444454) (end 83.525 97.525) (width 0.2) (layer "F.Cu") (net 2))
 (arc locked (start 84.625 97.525) (mid 84.819454 97.444454) (end 84.9 97.25) (width 0.2) (layer "F.Cu") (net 2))
 (arc (start 90.225 102.3068) (mid 90.144454 102.501254) (end 89.95 102.5818) (width 0.2) (layer "F.Cu") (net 2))
 (arc (start 89.5 104.7818) (mid 89.305546 104.862346) (end 89.225 105.0568) (width 0.2) (layer "F.Cu") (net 2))
 (arc locked (start 76.925 97.525) (mid 77.119454 97.444454) (end 77.2 97.25) (width 0.2) (layer "F.Cu") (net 2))
 (arc locked (start 76.1 96.8) (mid 76.180546 96.605546) (end 76.375 96.525) (width 0.2) (layer "F.Cu") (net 2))
 (arc locked (start 84.9 96.8) (mid 84.980546 96.605546) (end 85.175 96.525) (width 0.2) (layer "F.Cu") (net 2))
 (arc locked (start 81.875 96.525) (mid 82.069454 96.605546) (end 82.15 96.8) (width 0.2) (layer "F.Cu") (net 2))
 (arc locked (start 84.35 97.25) (mid 84.430546 97.444454) (end 84.625 97.525) (width 0.2) (layer "F.Cu") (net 2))
 (arc locked (start 84.075 96.525) (mid 84.269454 96.605546) (end 84.35 96.8) (width 0.2) (layer "F.Cu") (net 2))
 (arc (start 89.5 101.4818) (mid 89.305546 101.562346) (end 89.225 101.7568) (width 0.2) (layer "F.Cu") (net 2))
 (arc locked (start 79.675 96.525) (mid 79.869454 96.605546) (end 79.95 96.8) (width 0.2) (layer "F.Cu") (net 2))
 (arc (start 69.525 96.95) (mid 69.715381 96.490381) (end 70.175 96.3) (width 0.2) (layer "F.Cu") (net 2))
 (arc (start 67.425 98.55) (mid 67.483579 98.691421) (end 67.625 98.75) (width 0.2) (layer "F.Cu") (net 2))
 (arc (start 89.95 100.9318) (mid 90.144454 101.012346) (end 90.225 101.2068) (width 0.2) (layer "F.Cu") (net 2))
 (arc (start 87.969544 98.126039) (mid 88.163999 98.045494) (end 88.358453 98.12604) (width 0.2) (layer "F.Cu") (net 2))
 (arc locked (start 79.95 97.25) (mid 80.030546 97.444454) (end 80.225 97.525) (width 0.2) (layer "F.Cu") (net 2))
 (arc locked (start 78.025 97.525) (mid 78.219454 97.444454) (end 78.3 97.25) (width 0.2) (layer "F.Cu") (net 2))
 (arc locked (start 81.325 97.525) (mid 81.519454 97.444454) (end 81.6 97.25) (width 0.2) (layer "F.Cu") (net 2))
 (arc locked (start 82.425 97.525) (mid 82.619454 97.444454) (end 82.7 97.25) (width 0.2) (layer "F.Cu") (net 2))
 (arc (start 90.225 103.4068) (mid 90.144454 103.601254) (end 89.95 103.6818) (width 0.2) (layer "F.Cu") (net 2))
 (arc (start 89.225 100.6568) (mid 89.305546 100.851254) (end 89.5 100.9318) (width 0.2) (layer "F.Cu") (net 2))
 (arc locked (start 77.475 96.525) (mid 77.669454 96.605546) (end 77.75 96.8) (width 0.2) (layer "F.Cu") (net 2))
 (arc locked (start 76.375 96.525) (mid 76.569454 96.605546) (end 76.65 96.8) (width 0.2) (layer "F.Cu") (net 2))
 (arc (start 88.040254 99.222054) (mid 88.234709 99.302599) (end 88.429163 99.222053) (width 0.2) (layer "F.Cu") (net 2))
 (arc locked (start 79.4 96.8) (mid 79.480546 96.605546) (end 79.675 96.525) (width 0.2) (layer "F.Cu") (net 2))
 (arc locked (start 83.525 97.525) (mid 83.719454 97.444454) (end 83.8 97.25) (width 0.2) (layer "F.Cu") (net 2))
 (arc (start 88.358452 98.126039) (mid 88.438997 98.320494) (end 88.358451 98.514948) (width 0.2) (layer "F.Cu") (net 2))
 (arc locked (start 81.05 97.25) (mid 81.130546 97.444454) (end 81.325 97.525) (width 0.2) (layer "F.Cu") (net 2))
 (arc (start 69.125 98.55) (mid 69.183579 98.691421) (end 69.325 98.75) (width 0.2) (layer "F.Cu") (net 2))
 (arc locked (start 85.45 97.25) (mid 85.530546 97.444454) (end 85.725 97.525) (width 0.2) (layer "F.Cu") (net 2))
 (arc (start 69.325 98.75) (mid 69.466421 98.691421) (end 69.525 98.55) (width 0.2) (layer "F.Cu") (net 2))
 (arc locked (start 75.275 96.525) (mid 75.469454 96.605546) (end 75.55 96.8) (width 0.2) (layer "F.Cu") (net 2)))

